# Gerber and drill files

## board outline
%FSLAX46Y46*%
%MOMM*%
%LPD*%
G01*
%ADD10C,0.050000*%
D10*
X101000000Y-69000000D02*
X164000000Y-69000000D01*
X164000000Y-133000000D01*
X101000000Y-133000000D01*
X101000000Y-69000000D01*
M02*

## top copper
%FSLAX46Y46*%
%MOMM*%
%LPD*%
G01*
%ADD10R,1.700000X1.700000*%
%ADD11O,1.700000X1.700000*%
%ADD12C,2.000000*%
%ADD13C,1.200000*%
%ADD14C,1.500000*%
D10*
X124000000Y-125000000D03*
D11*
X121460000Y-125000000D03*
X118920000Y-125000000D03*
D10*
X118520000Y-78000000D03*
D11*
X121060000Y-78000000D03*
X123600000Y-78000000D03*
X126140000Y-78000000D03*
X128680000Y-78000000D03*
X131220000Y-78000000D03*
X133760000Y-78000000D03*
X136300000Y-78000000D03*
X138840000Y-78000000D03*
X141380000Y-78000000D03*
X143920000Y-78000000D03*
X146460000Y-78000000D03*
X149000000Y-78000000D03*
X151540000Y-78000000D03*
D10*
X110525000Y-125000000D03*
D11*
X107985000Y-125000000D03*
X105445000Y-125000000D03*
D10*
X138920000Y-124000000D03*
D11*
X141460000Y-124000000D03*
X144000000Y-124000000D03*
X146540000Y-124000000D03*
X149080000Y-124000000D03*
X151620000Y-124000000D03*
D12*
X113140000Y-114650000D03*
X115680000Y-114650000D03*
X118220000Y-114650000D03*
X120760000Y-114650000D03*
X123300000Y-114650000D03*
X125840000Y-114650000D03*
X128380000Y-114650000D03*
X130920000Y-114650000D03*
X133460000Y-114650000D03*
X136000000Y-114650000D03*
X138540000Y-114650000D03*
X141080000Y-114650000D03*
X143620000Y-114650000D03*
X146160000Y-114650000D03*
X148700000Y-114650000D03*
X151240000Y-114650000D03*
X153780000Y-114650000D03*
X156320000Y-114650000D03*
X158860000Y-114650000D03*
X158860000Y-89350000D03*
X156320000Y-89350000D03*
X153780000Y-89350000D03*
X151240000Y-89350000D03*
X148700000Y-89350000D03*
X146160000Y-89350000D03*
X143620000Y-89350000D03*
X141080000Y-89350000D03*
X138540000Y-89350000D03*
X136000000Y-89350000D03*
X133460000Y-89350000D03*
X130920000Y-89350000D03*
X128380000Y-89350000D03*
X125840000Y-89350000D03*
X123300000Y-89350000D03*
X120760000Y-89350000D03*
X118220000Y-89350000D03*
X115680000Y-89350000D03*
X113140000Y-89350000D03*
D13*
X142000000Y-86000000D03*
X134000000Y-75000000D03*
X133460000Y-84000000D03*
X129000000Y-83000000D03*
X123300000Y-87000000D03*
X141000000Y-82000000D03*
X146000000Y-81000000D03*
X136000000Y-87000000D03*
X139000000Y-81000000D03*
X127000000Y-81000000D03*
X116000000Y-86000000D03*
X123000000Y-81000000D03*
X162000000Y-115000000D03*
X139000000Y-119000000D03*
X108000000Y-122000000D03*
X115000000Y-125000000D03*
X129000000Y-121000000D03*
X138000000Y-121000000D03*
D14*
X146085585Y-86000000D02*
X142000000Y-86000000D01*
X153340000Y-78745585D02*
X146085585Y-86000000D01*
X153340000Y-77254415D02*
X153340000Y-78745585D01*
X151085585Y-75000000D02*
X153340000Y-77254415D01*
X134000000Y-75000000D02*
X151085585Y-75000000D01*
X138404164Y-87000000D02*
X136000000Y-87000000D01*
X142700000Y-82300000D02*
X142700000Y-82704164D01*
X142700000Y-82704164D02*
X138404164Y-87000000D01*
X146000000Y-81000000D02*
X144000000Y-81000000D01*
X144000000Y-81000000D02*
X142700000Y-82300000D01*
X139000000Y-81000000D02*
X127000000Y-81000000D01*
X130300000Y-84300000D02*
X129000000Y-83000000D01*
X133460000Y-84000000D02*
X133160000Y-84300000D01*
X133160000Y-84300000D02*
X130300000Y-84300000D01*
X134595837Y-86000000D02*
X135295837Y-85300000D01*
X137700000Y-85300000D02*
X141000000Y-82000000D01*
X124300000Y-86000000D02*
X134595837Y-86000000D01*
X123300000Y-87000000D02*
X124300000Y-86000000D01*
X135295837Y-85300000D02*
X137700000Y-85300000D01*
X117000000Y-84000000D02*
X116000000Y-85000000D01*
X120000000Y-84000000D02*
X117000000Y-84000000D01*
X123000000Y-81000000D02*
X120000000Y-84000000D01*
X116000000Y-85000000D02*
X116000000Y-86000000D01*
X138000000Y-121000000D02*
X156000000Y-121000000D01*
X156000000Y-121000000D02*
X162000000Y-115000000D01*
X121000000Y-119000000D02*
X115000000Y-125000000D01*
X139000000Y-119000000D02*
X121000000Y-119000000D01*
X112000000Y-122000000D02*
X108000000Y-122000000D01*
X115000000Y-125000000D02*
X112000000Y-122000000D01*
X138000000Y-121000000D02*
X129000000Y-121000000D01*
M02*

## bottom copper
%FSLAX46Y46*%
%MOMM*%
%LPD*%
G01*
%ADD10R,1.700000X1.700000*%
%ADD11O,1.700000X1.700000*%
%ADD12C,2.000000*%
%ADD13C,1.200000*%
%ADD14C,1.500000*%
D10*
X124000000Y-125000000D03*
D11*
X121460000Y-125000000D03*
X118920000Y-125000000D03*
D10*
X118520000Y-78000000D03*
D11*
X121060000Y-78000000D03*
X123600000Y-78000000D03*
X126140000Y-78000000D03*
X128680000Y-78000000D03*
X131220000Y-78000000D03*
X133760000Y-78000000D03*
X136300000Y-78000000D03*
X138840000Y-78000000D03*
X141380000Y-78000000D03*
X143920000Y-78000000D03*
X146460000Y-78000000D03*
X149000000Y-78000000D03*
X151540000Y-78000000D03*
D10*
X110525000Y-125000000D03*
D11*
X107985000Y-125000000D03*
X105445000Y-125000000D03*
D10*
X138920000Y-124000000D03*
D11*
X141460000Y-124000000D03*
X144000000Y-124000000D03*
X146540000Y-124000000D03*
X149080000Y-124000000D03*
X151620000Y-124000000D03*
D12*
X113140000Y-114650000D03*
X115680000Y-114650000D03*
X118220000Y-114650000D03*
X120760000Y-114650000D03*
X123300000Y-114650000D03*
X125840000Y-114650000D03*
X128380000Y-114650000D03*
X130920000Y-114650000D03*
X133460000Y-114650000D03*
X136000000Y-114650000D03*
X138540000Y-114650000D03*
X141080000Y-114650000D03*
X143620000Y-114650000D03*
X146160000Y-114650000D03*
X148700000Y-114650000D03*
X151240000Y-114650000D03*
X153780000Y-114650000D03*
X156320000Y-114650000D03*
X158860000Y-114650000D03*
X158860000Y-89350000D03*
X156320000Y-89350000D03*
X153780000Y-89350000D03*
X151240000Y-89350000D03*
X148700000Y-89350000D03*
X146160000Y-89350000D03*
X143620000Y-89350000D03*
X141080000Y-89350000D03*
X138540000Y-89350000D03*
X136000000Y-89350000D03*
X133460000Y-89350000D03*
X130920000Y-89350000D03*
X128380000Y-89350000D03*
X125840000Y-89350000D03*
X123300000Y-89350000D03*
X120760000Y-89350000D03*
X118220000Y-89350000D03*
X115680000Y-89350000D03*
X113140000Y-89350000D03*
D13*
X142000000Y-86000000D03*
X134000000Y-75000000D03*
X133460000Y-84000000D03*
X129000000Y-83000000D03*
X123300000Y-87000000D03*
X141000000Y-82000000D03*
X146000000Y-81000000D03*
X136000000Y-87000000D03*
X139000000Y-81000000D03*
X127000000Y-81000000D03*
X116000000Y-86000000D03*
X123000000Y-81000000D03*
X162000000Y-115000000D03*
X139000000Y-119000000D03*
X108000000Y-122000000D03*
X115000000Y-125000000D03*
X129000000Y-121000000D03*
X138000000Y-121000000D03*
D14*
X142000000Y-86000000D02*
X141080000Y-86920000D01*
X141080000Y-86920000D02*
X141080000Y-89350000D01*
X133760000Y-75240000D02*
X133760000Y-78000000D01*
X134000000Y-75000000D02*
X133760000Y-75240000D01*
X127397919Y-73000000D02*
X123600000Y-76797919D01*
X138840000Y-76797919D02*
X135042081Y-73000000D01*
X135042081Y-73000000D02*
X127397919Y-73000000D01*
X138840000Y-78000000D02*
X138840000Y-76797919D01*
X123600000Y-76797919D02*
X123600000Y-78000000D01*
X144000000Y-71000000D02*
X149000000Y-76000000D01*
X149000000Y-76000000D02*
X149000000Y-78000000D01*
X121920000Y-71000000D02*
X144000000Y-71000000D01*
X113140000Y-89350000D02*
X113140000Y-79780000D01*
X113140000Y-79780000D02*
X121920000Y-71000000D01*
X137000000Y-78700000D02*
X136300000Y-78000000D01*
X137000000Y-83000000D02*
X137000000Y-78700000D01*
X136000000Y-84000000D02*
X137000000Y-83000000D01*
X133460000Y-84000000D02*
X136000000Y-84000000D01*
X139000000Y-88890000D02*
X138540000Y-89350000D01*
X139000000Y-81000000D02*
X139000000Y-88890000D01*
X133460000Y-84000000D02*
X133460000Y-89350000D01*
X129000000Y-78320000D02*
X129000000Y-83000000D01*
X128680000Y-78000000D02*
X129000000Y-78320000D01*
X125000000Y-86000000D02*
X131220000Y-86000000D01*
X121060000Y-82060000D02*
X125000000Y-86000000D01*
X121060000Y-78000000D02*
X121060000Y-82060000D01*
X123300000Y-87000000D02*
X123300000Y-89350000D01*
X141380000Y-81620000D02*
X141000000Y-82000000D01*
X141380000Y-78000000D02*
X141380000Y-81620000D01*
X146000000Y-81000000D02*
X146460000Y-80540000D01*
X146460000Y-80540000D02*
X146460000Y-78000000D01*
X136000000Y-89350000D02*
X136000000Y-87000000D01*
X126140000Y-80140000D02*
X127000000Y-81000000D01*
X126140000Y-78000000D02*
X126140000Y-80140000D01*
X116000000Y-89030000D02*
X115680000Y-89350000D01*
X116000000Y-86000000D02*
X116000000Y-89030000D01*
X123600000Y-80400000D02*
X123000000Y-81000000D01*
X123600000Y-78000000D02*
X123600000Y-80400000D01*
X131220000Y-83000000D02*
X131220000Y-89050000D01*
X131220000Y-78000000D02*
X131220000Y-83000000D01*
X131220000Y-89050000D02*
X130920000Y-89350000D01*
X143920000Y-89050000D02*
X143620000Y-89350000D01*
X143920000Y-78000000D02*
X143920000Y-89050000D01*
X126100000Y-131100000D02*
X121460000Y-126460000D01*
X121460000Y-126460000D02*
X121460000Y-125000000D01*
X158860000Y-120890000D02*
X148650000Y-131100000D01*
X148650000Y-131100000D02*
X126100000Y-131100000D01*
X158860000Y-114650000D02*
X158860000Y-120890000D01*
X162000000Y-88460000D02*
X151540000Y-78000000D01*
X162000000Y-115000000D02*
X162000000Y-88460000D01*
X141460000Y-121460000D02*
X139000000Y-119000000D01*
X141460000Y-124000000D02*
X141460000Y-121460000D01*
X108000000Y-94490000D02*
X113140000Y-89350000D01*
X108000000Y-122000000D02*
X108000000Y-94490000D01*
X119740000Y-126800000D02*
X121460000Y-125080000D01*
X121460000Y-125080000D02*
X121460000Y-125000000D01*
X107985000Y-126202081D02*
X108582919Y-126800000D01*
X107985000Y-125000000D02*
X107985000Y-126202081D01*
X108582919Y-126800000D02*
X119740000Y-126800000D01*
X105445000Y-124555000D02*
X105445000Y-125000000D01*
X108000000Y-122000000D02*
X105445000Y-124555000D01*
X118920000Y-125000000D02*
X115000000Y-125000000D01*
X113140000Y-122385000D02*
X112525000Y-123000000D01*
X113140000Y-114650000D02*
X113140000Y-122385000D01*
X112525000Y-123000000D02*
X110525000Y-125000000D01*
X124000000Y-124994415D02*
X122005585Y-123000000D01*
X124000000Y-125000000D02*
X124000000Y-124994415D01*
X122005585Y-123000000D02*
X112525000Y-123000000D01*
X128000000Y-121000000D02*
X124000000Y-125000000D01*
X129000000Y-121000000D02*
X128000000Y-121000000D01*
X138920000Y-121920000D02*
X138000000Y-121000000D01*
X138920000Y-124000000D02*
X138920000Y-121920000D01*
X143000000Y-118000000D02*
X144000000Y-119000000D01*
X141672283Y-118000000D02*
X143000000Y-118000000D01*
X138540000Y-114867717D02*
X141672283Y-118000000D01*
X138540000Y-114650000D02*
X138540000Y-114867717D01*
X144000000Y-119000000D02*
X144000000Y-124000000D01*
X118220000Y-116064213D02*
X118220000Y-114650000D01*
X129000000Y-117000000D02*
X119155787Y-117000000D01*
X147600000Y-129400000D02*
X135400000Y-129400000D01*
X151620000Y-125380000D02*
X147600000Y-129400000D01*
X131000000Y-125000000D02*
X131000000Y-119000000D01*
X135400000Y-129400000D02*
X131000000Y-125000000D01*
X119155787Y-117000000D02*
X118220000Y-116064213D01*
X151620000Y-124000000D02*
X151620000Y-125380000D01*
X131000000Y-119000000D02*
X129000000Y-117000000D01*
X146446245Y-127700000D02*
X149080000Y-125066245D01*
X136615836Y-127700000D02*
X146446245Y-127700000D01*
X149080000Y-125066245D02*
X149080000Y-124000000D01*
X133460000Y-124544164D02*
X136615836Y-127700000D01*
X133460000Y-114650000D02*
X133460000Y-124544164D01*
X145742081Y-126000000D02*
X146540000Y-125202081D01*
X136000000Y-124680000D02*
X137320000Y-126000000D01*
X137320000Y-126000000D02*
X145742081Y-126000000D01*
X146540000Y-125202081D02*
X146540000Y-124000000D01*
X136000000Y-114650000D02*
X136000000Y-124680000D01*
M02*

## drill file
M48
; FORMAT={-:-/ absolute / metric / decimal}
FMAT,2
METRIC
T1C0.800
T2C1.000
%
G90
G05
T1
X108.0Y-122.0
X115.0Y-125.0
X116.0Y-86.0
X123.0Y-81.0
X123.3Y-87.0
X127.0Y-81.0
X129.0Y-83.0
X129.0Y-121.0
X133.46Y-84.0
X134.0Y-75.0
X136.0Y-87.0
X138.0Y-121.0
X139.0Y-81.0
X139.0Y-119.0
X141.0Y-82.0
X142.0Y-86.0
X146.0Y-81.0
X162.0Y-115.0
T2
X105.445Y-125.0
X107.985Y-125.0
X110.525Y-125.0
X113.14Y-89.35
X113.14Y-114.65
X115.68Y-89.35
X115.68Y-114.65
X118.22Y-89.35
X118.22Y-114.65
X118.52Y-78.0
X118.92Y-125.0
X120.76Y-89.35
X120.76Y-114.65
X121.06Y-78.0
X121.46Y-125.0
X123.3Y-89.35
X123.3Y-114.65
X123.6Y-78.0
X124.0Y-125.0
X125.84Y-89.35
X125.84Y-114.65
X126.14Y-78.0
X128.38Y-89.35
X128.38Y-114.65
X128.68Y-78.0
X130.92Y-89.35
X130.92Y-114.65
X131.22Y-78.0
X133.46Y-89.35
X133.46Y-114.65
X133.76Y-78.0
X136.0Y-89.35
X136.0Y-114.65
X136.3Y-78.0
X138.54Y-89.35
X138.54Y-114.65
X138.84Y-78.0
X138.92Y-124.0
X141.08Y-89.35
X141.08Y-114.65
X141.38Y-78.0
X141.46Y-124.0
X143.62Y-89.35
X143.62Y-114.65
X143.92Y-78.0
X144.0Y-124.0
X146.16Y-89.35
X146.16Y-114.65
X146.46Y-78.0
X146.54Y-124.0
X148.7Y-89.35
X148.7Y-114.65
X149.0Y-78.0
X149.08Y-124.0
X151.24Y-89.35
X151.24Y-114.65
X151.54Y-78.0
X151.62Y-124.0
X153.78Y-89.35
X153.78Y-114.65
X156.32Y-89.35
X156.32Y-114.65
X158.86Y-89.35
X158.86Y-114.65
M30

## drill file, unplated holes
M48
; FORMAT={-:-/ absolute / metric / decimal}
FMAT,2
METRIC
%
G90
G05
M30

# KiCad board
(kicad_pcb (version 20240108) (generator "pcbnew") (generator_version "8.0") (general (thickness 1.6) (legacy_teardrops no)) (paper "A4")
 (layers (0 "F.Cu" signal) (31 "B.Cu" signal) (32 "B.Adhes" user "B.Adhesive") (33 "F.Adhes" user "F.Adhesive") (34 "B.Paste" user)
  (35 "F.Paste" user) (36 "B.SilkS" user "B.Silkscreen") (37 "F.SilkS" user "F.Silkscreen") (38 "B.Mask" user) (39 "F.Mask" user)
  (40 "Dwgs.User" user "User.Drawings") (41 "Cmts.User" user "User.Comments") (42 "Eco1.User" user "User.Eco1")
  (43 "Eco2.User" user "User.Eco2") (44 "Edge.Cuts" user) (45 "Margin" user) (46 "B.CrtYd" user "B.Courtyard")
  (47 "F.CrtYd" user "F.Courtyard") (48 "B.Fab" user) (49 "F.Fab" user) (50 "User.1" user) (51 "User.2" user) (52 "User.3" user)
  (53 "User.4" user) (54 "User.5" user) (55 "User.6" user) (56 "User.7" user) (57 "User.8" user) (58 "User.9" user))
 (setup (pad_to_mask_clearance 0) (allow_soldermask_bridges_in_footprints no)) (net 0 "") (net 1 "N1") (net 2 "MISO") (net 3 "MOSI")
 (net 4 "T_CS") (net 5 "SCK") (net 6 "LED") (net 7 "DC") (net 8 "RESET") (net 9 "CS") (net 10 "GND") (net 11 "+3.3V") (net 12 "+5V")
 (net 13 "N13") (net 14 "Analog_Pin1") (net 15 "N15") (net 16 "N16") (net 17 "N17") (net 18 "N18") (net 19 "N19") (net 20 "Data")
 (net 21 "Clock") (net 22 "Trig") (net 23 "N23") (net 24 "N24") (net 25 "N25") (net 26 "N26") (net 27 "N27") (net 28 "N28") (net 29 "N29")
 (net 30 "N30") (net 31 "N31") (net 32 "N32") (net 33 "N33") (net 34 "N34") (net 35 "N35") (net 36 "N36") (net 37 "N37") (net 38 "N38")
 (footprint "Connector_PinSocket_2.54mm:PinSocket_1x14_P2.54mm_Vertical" (layer "F.Cu") (at 118.52 78 90)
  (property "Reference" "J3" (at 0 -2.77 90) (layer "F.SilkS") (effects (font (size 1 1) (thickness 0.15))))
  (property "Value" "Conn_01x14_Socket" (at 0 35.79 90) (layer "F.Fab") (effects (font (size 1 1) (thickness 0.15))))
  (pad "1" thru_hole rect (at 0 0 90) (size 1.7 1.7) (drill 1) (layers "*.Cu" "*.Mask") (remove_unused_layers no) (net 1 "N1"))
  (pad "2" thru_hole oval (at 0 2.54 90) (size 1.7 1.7) (drill 1) (layers "*.Cu" "*.Mask") (remove_unused_layers no) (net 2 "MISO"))
  (pad "3" thru_hole oval (at 0 5.08 90) (size 1.7 1.7) (drill 1) (layers "*.Cu" "*.Mask") (remove_unused_layers no) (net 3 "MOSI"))
  (pad "4" thru_hole oval (at 0 7.62 90) (size 1.7 1.7) (drill 1) (layers "*.Cu" "*.Mask") (remove_unused_layers no) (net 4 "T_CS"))
  (pad "5" thru_hole oval (at 0 10.16 90) (size 1.7 1.7) (drill 1) (layers "*.Cu" "*.Mask") (remove_unused_layers no) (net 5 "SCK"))
  (pad "6" thru_hole oval (at 0 12.7 90) (size 1.7 1.7) (drill 1) (layers "*.Cu" "*.Mask") (remove_unused_layers no) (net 2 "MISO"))
  (pad "7" thru_hole oval (at 0 15.24 90) (size 1.7 1.7) (drill 1) (layers "*.Cu" "*.Mask") (remove_unused_layers no) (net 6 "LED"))
  (pad "8" thru_hole oval (at 0 17.78 90) (size 1.7 1.7) (drill 1) (layers "*.Cu" "*.Mask") (remove_unused_layers no) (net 5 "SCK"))
  (pad "9" thru_hole oval (at 0 20.32 90) (size 1.7 1.7) (drill 1) (layers "*.Cu" "*.Mask") (remove_unused_layers no) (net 3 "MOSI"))
  (pad "10" thru_hole oval (at 0 22.86 90) (size 1.7 1.7) (drill 1) (layers "*.Cu" "*.Mask") (remove_unused_layers no) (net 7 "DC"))
  (pad "11" thru_hole oval (at 0 25.4 90) (size 1.7 1.7) (drill 1) (layers "*.Cu" "*.Mask") (remove_unused_layers no) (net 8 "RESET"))
  (pad "12" thru_hole oval (at 0 27.94 90) (size 1.7 1.7) (drill 1) (layers "*.Cu" "*.Mask") (remove_unused_layers no) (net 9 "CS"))
  (pad "13" thru_hole oval (at 0 30.48 90) (size 1.7 1.7) (drill 1) (layers "*.Cu" "*.Mask") (remove_unused_layers no) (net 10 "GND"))
  (pad "14" thru_hole oval (at 0 33.02 90) (size 1.7 1.7) (drill 1) (layers "*.Cu" "*.Mask") (remove_unused_layers no) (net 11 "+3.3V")))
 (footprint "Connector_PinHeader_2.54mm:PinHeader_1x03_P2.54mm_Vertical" (layer "F.Cu") (at 124 125 -90)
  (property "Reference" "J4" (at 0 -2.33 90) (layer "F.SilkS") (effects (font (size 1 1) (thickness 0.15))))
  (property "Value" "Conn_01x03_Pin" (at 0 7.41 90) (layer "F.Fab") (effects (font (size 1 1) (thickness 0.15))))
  (pad "1" thru_hole rect (at 0 0 270) (size 1.7 1.7) (drill 1) (layers "*.Cu" "*.Mask") (remove_unused_layers no) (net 11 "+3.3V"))
  (pad "2" thru_hole oval (at 0 2.54 270) (size 1.7 1.7) (drill 1) (layers "*.Cu" "*.Mask") (remove_unused_layers no) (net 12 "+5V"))
  (pad "3" thru_hole oval (at 0 5.08 270) (size 1.7 1.7) (drill 1) (layers "*.Cu" "*.Mask") (remove_unused_layers no) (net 10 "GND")))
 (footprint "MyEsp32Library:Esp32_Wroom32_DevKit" (layer "F.Cu") (at 136 102)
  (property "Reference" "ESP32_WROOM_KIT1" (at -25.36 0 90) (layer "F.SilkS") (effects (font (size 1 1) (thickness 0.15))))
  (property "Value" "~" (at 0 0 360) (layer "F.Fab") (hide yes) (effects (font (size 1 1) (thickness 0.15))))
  (pad "1" thru_hole circle (at -22.86 12.65) (size 2 2) (drill 1) (layers "*.Cu" "*.Mask") (remove_unused_layers no) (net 11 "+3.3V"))
  (pad "2" thru_hole circle (at -20.32 12.65) (size 2 2) (drill 1) (layers "*.Cu" "*.Mask") (remove_unused_layers no) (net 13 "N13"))
  (pad "3" thru_hole circle (at -17.78 12.65) (size 2 2) (drill 1) (layers "*.Cu" "*.Mask") (remove_unused_layers no) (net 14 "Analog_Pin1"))
  (pad "4" thru_hole circle (at -15.24 12.65) (size 2 2) (drill 1) (layers "*.Cu" "*.Mask") (remove_unused_layers no) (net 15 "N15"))
  (pad "5" thru_hole circle (at -12.7 12.65) (size 2 2) (drill 1) (layers "*.Cu" "*.Mask") (remove_unused_layers no) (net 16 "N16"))
  (pad "6" thru_hole circle (at -10.16 12.65) (size 2 2) (drill 1) (layers "*.Cu" "*.Mask") (remove_unused_layers no) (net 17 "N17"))
  (pad "7" thru_hole circle (at -7.62 12.65) (size 2 2) (drill 1) (layers "*.Cu" "*.Mask") (remove_unused_layers no) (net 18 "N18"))
  (pad "8" thru_hole circle (at -5.08 12.65) (size 2 2) (drill 1) (layers "*.Cu" "*.Mask") (remove_unused_layers no) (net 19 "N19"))
  (pad "9" thru_hole circle (at -2.54 12.65) (size 2 2) (drill 1) (layers "*.Cu" "*.Mask") (remove_unused_layers no) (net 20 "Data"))
  (pad "10" thru_hole circle (at 0 12.65) (size 2 2) (drill 1) (layers "*.Cu" "*.Mask") (remove_unused_layers no) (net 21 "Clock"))
  (pad "11" thru_hole circle (at 2.54 12.65) (size 2 2) (drill 1) (layers "*.Cu" "*.Mask") (remove_unused_layers no) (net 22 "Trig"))
  (pad "12" thru_hole circle (at 5.08 12.65) (size 2 2) (drill 1) (layers "*.Cu" "*.Mask") (remove_unused_layers no) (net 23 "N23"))
  (pad "13" thru_hole circle (at 7.62 12.65) (size 2 2) (drill 1) (layers "*.Cu" "*.Mask") (remove_unused_layers no) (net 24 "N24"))
  (pad "14" thru_hole circle (at 10.16 12.65) (size 2 2) (drill 1) (layers "*.Cu" "*.Mask") (remove_unused_layers no) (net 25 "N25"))
  (pad "15" thru_hole circle (at 12.7 12.65) (size 2 2) (drill 1) (layers "*.Cu" "*.Mask") (remove_unused_layers no) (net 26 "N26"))
  (pad "16" thru_hole circle (at 15.24 12.65) (size 2 2) (drill 1) (layers "*.Cu" "*.Mask") (remove_unused_layers no) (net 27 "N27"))
  (pad "17" thru_hole circle (at 17.78 12.65) (size 2 2) (drill 1) (layers "*.Cu" "*.Mask") (remove_unused_layers no) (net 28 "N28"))
  (pad "18" thru_hole circle (at 20.32 12.65) (size 2 2) (drill 1) (layers "*.Cu" "*.Mask") (remove_unused_layers no) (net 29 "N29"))
  (pad "19" thru_hole circle (at 22.86 12.65) (size 2 2) (drill 1) (layers "*.Cu" "*.Mask") (remove_unused_layers no) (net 12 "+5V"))
  (pad "20" thru_hole circle (at 22.86 -12.65) (size 2 2) (drill 1) (layers "*.Cu" "*.Mask") (remove_unused_layers no) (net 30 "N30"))
  (pad "21" thru_hole circle (at 20.32 -12.65) (size 2 2) (drill 1) (layers "*.Cu" "*.Mask") (remove_unused_layers no) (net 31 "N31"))
  (pad "22" thru_hole circle (at 17.78 -12.65) (size 2 2) (drill 1) (layers "*.Cu" "*.Mask") (remove_unused_layers no) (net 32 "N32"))
  (pad "23" thru_hole circle (at 15.24 -12.65) (size 2 2) (drill 1) (layers "*.Cu" "*.Mask") (remove_unused_layers no) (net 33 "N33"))
  (pad "24" thru_hole circle (at 12.7 -12.65) (size 2 2) (drill 1) (layers "*.Cu" "*.Mask") (remove_unused_layers no))
  (pad "25" thru_hole circle (at 10.16 -12.65) (size 2 2) (drill 1) (layers "*.Cu" "*.Mask") (remove_unused_layers no) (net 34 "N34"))
  (pad "26" thru_hole circle (at 7.62 -12.65) (size 2 2) (drill 1) (layers "*.Cu" "*.Mask") (remove_unused_layers no) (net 8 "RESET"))
  (pad "27" thru_hole circle (at 5.08 -12.65) (size 2 2) (drill 1) (layers "*.Cu" "*.Mask") (remove_unused_layers no) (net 6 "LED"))
  (pad "28" thru_hole circle (at 2.54 -12.65) (size 2 2) (drill 1) (layers "*.Cu" "*.Mask") (remove_unused_layers no) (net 4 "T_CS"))
  (pad "29" thru_hole circle (at 0 -12.65) (size 2 2) (drill 1) (layers "*.Cu" "*.Mask") (remove_unused_layers no) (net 9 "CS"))
  (pad "30" thru_hole circle (at -2.54 -12.65) (size 2 2) (drill 1) (layers "*.Cu" "*.Mask") (remove_unused_layers no) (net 5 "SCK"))
  (pad "31" thru_hole circle (at -5.08 -12.65) (size 2 2) (drill 1) (layers "*.Cu" "*.Mask") (remove_unused_layers no) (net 2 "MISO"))
  (pad "32" thru_hole circle (at -7.62 -12.65) (size 2 2) (drill 1) (layers "*.Cu" "*.Mask") (remove_unused_layers no) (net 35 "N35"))
  (pad "33" thru_hole circle (at -10.16 -12.65) (size 2 2) (drill 1) (layers "*.Cu" "*.Mask") (remove_unused_layers no) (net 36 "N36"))
  (pad "34" thru_hole circle (at -12.7 -12.65) (size 2 2) (drill 1) (layers "*.Cu" "*.Mask") (remove_unused_layers no) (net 7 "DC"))
  (pad "35" thru_hole circle (at -15.24 -12.65) (size 2 2) (drill 1) (layers "*.Cu" "*.Mask") (remove_unused_layers no) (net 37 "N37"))
  (pad "36" thru_hole circle (at -17.78 -12.65) (size 2 2) (drill 1) (layers "*.Cu" "*.Mask") (remove_unused_layers no) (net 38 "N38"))
  (pad "37" thru_hole circle (at -20.32 -12.65) (size 2 2) (drill 1) (layers "*.Cu" "*.Mask") (remove_unused_layers no) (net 3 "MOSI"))
  (pad "38" thru_hole circle (at -22.86 -12.65) (size 2 2) (drill 1) (layers "*.Cu" "*.Mask") (remove_unused_layers no) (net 10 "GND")))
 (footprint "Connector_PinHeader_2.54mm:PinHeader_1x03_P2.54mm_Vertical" (layer "F.Cu") (at 110.525 125 -90)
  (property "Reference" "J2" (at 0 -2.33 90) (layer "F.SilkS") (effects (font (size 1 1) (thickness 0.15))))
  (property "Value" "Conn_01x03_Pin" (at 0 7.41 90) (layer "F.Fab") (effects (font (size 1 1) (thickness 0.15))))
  (pad "1" thru_hole rect (at 0 0 270) (size 1.7 1.7) (drill 1) (layers "*.Cu" "*.Mask") (remove_unused_layers no) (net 11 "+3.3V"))
  (pad "2" thru_hole oval (at 0 2.54 270) (size 1.7 1.7) (drill 1) (layers "*.Cu" "*.Mask") (remove_unused_layers no) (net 12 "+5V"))
  (pad "3" thru_hole oval (at 0 5.08 270) (size 1.7 1.7) (drill 1) (layers "*.Cu" "*.Mask") (remove_unused_layers no) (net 10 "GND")))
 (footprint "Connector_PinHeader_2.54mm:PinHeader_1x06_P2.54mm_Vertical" (layer "F.Cu") (at 138.92 124 90)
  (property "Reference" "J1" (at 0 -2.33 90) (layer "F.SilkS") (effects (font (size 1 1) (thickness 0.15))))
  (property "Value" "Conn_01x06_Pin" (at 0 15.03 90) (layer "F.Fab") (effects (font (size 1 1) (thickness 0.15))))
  (pad "1" thru_hole rect (at 0 0 90) (size 1.7 1.7) (drill 1) (layers "*.Cu" "*.Mask") (remove_unused_layers no) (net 11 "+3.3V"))
  (pad "2" thru_hole oval (at 0 2.54 90) (size 1.7 1.7) (drill 1) (layers "*.Cu" "*.Mask") (remove_unused_layers no) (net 10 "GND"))
  (pad "3" thru_hole oval (at 0 5.08 90) (size 1.7 1.7) (drill 1) (layers "*.Cu" "*.Mask") (remove_unused_layers no) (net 22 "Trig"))
  (pad "4" thru_hole oval (at 0 7.62 90) (size 1.7 1.7) (drill 1) (layers "*.Cu" "*.Mask") (remove_unused_layers no) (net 21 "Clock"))
  (pad "5" thru_hole oval (at 0 10.16 90) (size 1.7 1.7) (drill 1) (layers "*.Cu" "*.Mask") (remove_unused_layers no) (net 20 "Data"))
  (pad "6" thru_hole oval (at 0 12.7 90) (size 1.7 1.7) (drill 1) (layers "*.Cu" "*.Mask") (remove_unused_layers no) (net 14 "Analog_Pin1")))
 (gr_rect (start 101 69) (end 164 133) (stroke (width 0.05) (type default)) (fill none) (layer "Edge.Cuts"))
 (segment (start 123 81) (end 120 84) (width 1.5) (layer "F.Cu") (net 3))
 (segment (start 117 84) (end 116 85) (width 1.5) (layer "F.Cu") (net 3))
 (segment (start 116 85) (end 116 86) (width 1.5) (layer "F.Cu") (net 3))
 (segment (start 120 84) (end 117 84) (width 1.5) (layer "F.Cu") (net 3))
 (via (at 123 81) (size 1.2) (drill 0.8) (layers "F.Cu" "B.Cu") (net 3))
 (via (at 116 86) (size 1.2) (drill 0.8) (layers "F.Cu" "B.Cu") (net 3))
 (segment (start 138.84 76.797919) (end 135.042081 73) (width 1.5) (layer "B.Cu") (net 3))
 (segment (start 123.6 80.4) (end 123 81) (width 1.5) (layer "B.Cu") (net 3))
 (segment (start 138.84 78) (end 138.84 76.797919) (width 1.5) (layer "B.Cu") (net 3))
 (segment (start 123.6 76.797919) (end 123.6 78) (width 1.5) (layer "B.Cu") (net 3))
 (segment (start 127.397919 73) (end 123.6 76.797919) (width 1.5) (layer "B.Cu") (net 3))
 (segment (start 123.6 78) (end 123.6 80.4) (width 1.5) (layer "B.Cu") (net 3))
 (segment (start 135.042081 73) (end 127.397919 73) (width 1.5) (layer "B.Cu") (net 3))
 (segment (start 116 86) (end 116 89.03) (width 1.5) (layer "B.Cu") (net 3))
 (segment (start 116 89.03) (end 115.68 89.35) (width 1.5) (layer "B.Cu") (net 3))
 (segment (start 115 125) (end 112 122) (width 1.5) (layer "F.Cu") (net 10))
 (segment (start 121 119) (end 115 125) (width 1.5) (layer "F.Cu") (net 10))
 (segment (start 139 119) (end 121 119) (width 1.5) (layer "F.Cu") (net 10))
 (segment (start 112 122) (end 108 122) (width 1.5) (layer "F.Cu") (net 10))
 (via (at 139 119) (size 1.2) (drill 0.8) (layers "F.Cu" "B.Cu") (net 10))
 (via (at 115 125) (size 1.2) (drill 0.8) (layers "F.Cu" "B.Cu") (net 10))
 (via (at 108 122) (size 1.2) (drill 0.8) (layers "F.Cu" "B.Cu") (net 10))
 (segment (start 113.14 89.35) (end 113.14 79.78) (width 1.5) (layer "B.Cu") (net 10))
 (segment (start 105.445 124.555) (end 105.445 125) (width 1.5) (layer "B.Cu") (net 10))
 (segment (start 121.92 71) (end 144 71) (width 1.5) (layer "B.Cu") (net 10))
 (segment (start 149 76) (end 149 78) (width 1.5) (layer "B.Cu") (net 10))
 (segment (start 118.92 125) (end 115 125) (width 1.5) (layer "B.Cu") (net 10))
 (segment (start 113.14 79.78) (end 121.92 71) (width 1.5) (layer "B.Cu") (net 10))
 (segment (start 108 122) (end 108 94.49) (width 1.5) (layer "B.Cu") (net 10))
 (segment (start 108 122) (end 105.445 124.555) (width 1.5) (layer "B.Cu") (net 10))
 (segment (start 141.46 121.46) (end 139 119) (width 1.5) (layer "B.Cu") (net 10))
 (segment (start 144 71) (end 149 76) (width 1.5) (layer "B.Cu") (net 10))
 (segment (start 141.46 124) (end 141.46 121.46) (width 1.5) (layer "B.Cu") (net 10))
 (segment (start 108 94.49) (end 113.14 89.35) (width 1.5) (layer "B.Cu") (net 10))
 (segment (start 138 121) (end 156 121) (width 1.5) (layer "F.Cu") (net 11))
 (segment (start 138 121) (end 129 121) (width 1.5) (layer "F.Cu") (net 11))
 (segment (start 156 121) (end 162 115) (width 1.5) (layer "F.Cu") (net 11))
 (via (at 138 121) (size 1.2) (drill 0.8) (layers "F.Cu" "B.Cu") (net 11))
 (via (at 129 121) (size 1.2) (drill 0.8) (layers "F.Cu" "B.Cu") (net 11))
 (via (at 162 115) (size 1.2) (drill 0.8) (layers "F.Cu" "B.Cu") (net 11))
 (segment (start 122.005585 123) (end 112.525 123) (width 1.5) (layer "B.Cu") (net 11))
 (segment (start 124 125) (end 124 124.994415) (width 1.5) (layer "B.Cu") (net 11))
 (segment (start 138.92 121.92) (end 138 121) (width 1.5) (layer "B.Cu") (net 11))
 (segment (start 112.525 123) (end 110.525 125) (width 1.5) (layer "B.Cu") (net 11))
 (segment (start 124 124.994415) (end 122.005585 123) (width 1.5) (layer "B.Cu") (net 11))
 (segment (start 113.14 122.385) (end 112.525 123) (width 1.5) (layer "B.Cu") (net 11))
 (segment (start 138.92 124) (end 138.92 121.92) (width 1.5) (layer "B.Cu") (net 11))
 (segment (start 162 115) (end 162 88.46) (width 1.5) (layer "B.Cu") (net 11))
 (segment (start 162 88.46) (end 151.54 78) (width 1.5) (layer "B.Cu") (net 11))
 (segment (start 129 121) (end 128 121) (width 1.5) (layer "B.Cu") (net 11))
 (segment (start 113.14 114.65) (end 113.14 122.385) (width 1.5) (layer "B.Cu") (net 11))
 (segment (start 128 121) (end 124 125) (width 1.5) (layer "B.Cu") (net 11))
 (segment (start 130.3 84.3) (end 129 83) (width 1.5) (layer "F.Cu") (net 5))
 (segment (start 133.16 84.3) (end 130.3 84.3) (width 1.5) (layer "F.Cu") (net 5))
 (segment (start 133.46 84) (end 133.16 84.3) (width 1.5) (layer "F.Cu") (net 5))
 (via (at 133.46 84) (size 1.2) (drill 0.8) (layers "F.Cu" "B.Cu") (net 5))
 (via (at 129 83) (size 1.2) (drill 0.8) (layers "F.Cu" "B.Cu") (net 5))
 (segment (start 133.46 84) (end 136 84) (width 1.5) (layer "B.Cu") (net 5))
 (segment (start 137 78.7) (end 136.3 78) (width 1.5) (layer "B.Cu") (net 5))
 (segment (start 137 83) (end 137 78.7) (width 1.5) (layer "B.Cu") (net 5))
 (segment (start 136 84) (end 137 83) (width 1.5) (layer "B.Cu") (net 5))
 (segment (start 128.68 78) (end 129 78.32) (width 1.5) (layer "B.Cu") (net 5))
 (segment (start 133.46 84) (end 133.46 89.35) (width 1.5) (layer "B.Cu") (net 5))
 (segment (start 129 78.32) (end 129 83) (width 1.5) (layer "B.Cu") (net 5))
 (segment (start 146 81) (end 144 81) (width 1.5) (layer "F.Cu") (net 9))
 (segment (start 142.7 82.704164) (end 138.404164 87) (width 1.5) (layer "F.Cu") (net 9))
 (segment (start 142.7 82.3) (end 142.7 82.704164) (width 1.5) (layer "F.Cu") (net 9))
 (segment (start 144 81) (end 142.7 82.3) (width 1.5) (layer "F.Cu") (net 9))
 (segment (start 138.404164 87) (end 136 87) (width 1.5) (layer "F.Cu") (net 9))
 (via (at 136 87) (size 1.2) (drill 0.8) (layers "F.Cu" "B.Cu") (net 9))
 (via (at 146 81) (size 1.2) (drill 0.8) (layers "F.Cu" "B.Cu") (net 9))
 (segment (start 136 89.35) (end 136 87) (width 1.5) (layer "B.Cu") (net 9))
 (segment (start 146 81) (end 146.46 80.54) (width 1.5) (layer "B.Cu") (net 9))
 (segment (start 146.46 80.54) (end 146.46 78) (width 1.5) (layer "B.Cu") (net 9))
 (segment (start 143 118) (end 144 119) (width 1.5) (layer "B.Cu") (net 22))
 (segment (start 138.54 114.65) (end 138.54 114.867717) (width 1.5) (layer "B.Cu") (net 22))
 (segment (start 138.54 114.867717) (end 141.672283 118) (width 1.5) (layer "B.Cu") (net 22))
 (segment (start 144 119) (end 144 124) (width 1.5) (layer "B.Cu") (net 22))
 (segment (start 141.672283 118) (end 143 118) (width 1.5) (layer "B.Cu") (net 22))
 (segment (start 133.46 114.65) (end 133.46 124.544164) (width 1.5) (layer "B.Cu") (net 20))
 (segment (start 146.446245 127.7) (end 149.08 125.066245) (width 1.5) (layer "B.Cu") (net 20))
 (segment (start 133.46 124.544164) (end 136.615836 127.7) (width 1.5) (layer "B.Cu") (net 20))
 (segment (start 136.615836 127.7) (end 146.446245 127.7) (width 1.5) (layer "B.Cu") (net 20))
 (segment (start 149.08 125.066245) (end 149.08 124) (width 1.5) (layer "B.Cu") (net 20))
 (segment (start 143.92 78) (end 143.92 89.05) (width 1.5) (layer "B.Cu") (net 8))
 (segment (start 143.92 89.05) (end 143.62 89.35) (width 1.5) (layer "B.Cu") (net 8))
 (segment (start 108.582919 126.8) (end 119.74 126.8) (width 1.5) (layer "B.Cu") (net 12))
 (segment (start 121.46 126.46) (end 121.46 125) (width 1.5) (layer "B.Cu") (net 12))
 (segment (start 126.1 131.1) (end 121.46 126.46) (width 1.5) (layer "B.Cu") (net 12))
 (segment (start 148.65 131.1) (end 126.1 131.1) (width 1.5) (layer "B.Cu") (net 12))
 (segment (start 158.86 114.65) (end 158.86 120.89) (width 1.5) (layer "B.Cu") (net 12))
 (segment (start 107.985 125) (end 107.985 126.202081) (width 1.5) (layer "B.Cu") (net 12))
 (segment (start 119.74 126.8) (end 121.46 125.08) (width 1.5) (layer "B.Cu") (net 12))
 (segment (start 107.985 126.202081) (end 108.582919 126.8) (width 1.5) (layer "B.Cu") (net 12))
 (segment (start 121.46 125.08) (end 121.46 125) (width 1.5) (layer "B.Cu") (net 12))
 (segment (start 158.86 120.89) (end 148.65 131.1) (width 1.5) (layer "B.Cu") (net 12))
 (segment (start 131 125) (end 131 119) (width 1.5) (layer "B.Cu") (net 14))
 (segment (start 151.62 124) (end 151.62 125.38) (width 1.5) (layer "B.Cu") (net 14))
 (segment (start 147.6 129.4) (end 135.4 129.4) (width 1.5) (layer "B.Cu") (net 14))
 (segment (start 135.4 129.4) (end 131 125) (width 1.5) (layer "B.Cu") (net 14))
 (segment (start 151.62 125.38) (end 147.6 129.4) (width 1.5) (layer "B.Cu") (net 14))
 (segment (start 119.155787 117) (end 118.22 116.064213) (width 1.5) (layer "B.Cu") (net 14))
 (segment (start 118.22 116.064213) (end 118.22 114.65) (width 1.5) (layer "B.Cu") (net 14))
 (segment (start 131 119) (end 129 117) (width 1.5) (layer "B.Cu") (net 14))
 (segment (start 129 117) (end 119.155787 117) (width 1.5) (layer "B.Cu") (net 14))
 (segment (start 145.742081 126) (end 146.54 125.202081) (width 1.5) (layer "B.Cu") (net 21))
 (segment (start 136 114.65) (end 136 124.68) (width 1.5) (layer "B.Cu") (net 21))
 (segment (start 137.32 126) (end 145.742081 126) (width 1.5) (layer "B.Cu") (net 21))
 (segment (start 136 124.68) (end 137.32 126) (width 1.5) (layer "B.Cu") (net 21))
 (segment (start 146.54 125.202081) (end 146.54 124) (width 1.5) (layer "B.Cu") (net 21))
 (segment (start 124.3 86) (end 134.595837 86) (width 1.5) (layer "F.Cu") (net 7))
 (segment (start 137.7 85.3) (end 141 82) (width 1.5) (layer "F.Cu") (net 7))
 (segment (start 135.295837 85.3) (end 137.7 85.3) (width 1.5) (layer "F.Cu") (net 7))
 (segment (start 134.595837 86) (end 135.295837 85.3) (width 1.5) (layer "F.Cu") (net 7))
 (segment (start 123.3 87) (end 124.3 86) (width 1.5) (layer "F.Cu") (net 7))
 (via (at 123.3 87) (size 1.2) (drill 0.8) (layers "F.Cu" "B.Cu") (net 7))
 (via (at 141 82) (size 1.2) (drill 0.8) (layers "F.Cu" "B.Cu") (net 7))
 (segment (start 141.38 78) (end 141.38 81.62) (width 1.5) (layer "B.Cu") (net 7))
 (segment (start 141.38 81.62) (end 141 82) (width 1.5) (layer "B.Cu") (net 7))
 (segment (start 123.3 87) (end 123.3 89.35) (width 1.5) (layer "B.Cu") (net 7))
 (segment (start 125 86) (end 131.22 86) (width 1.5) (layer "B.Cu") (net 2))
 (segment (start 121.06 78) (end 121.06 82.06) (width 1.5) (layer "B.Cu") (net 2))
 (segment (start 121.06 82.06) (end 125 86) (width 1.5) (layer "B.Cu") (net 2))
 (segment (start 131.22 89.05) (end 130.92 89.35) (width 1.5) (layer "B.Cu") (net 2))
 (segment (start 131.22 83) (end 131.22 89.05) (width 1.5) (layer "B.Cu") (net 2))
 (segment (start 131.22 78) (end 131.22 83) (width 1.5) (layer "B.Cu") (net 2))
 (segment (start 146.085585 86) (end 142 86) (width 1.5) (layer "F.Cu") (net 6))
 (segment (start 153.34 78.745585) (end 146.085585 86) (width 1.5) (layer "F.Cu") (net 6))
 (segment (start 151.085585 75) (end 153.34 77.254415) (width 1.5) (layer "F.Cu") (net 6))
 (segment (start 153.34 77.254415) (end 153.34 78.745585) (width 1.5) (layer "F.Cu") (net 6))
 (segment (start 134 75) (end 151.085585 75) (width 1.5) (layer "F.Cu") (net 6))
 (via (at 134 75) (size 1.2) (drill 0.8) (layers "F.Cu" "B.Cu") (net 6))
 (via (at 142 86) (size 1.2) (drill 0.8) (layers "F.Cu" "B.Cu") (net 6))
 (segment (start 134 75) (end 133.76 75.24) (width 1.5) (layer "B.Cu") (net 6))
 (segment (start 141.08 86.92) (end 141.08 89.35) (width 1.5) (layer "B.Cu") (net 6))
 (segment (start 142 86) (end 141.08 86.92) (width 1.5) (layer "B.Cu") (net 6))
 (segment (start 133.76 75.24) (end 133.76 78) (width 1.5) (layer "B.Cu") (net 6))
 (segment (start 139 81) (end 127 81) (width 1.5) (layer "F.Cu") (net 4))
 (via (at 139 81) (size 1.2) (drill 0.8) (layers "F.Cu" "B.Cu") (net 4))
 (via (at 127 81) (size 1.2) (drill 0.8) (layers "F.Cu" "B.Cu") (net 4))
 (segment (start 139 88.89) (end 138.54 89.35) (width 1.5) (layer "B.Cu") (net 4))
 (segment (start 126.14 80.14) (end 127 81) (width 1.5) (layer "B.Cu") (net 4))
 (segment (start 126.14 78) (end 126.14 80.14) (width 1.5) (layer "B.Cu") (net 4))
 (segment (start 139 81) (end 139 88.89) (width 1.5) (layer "B.Cu") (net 4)))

